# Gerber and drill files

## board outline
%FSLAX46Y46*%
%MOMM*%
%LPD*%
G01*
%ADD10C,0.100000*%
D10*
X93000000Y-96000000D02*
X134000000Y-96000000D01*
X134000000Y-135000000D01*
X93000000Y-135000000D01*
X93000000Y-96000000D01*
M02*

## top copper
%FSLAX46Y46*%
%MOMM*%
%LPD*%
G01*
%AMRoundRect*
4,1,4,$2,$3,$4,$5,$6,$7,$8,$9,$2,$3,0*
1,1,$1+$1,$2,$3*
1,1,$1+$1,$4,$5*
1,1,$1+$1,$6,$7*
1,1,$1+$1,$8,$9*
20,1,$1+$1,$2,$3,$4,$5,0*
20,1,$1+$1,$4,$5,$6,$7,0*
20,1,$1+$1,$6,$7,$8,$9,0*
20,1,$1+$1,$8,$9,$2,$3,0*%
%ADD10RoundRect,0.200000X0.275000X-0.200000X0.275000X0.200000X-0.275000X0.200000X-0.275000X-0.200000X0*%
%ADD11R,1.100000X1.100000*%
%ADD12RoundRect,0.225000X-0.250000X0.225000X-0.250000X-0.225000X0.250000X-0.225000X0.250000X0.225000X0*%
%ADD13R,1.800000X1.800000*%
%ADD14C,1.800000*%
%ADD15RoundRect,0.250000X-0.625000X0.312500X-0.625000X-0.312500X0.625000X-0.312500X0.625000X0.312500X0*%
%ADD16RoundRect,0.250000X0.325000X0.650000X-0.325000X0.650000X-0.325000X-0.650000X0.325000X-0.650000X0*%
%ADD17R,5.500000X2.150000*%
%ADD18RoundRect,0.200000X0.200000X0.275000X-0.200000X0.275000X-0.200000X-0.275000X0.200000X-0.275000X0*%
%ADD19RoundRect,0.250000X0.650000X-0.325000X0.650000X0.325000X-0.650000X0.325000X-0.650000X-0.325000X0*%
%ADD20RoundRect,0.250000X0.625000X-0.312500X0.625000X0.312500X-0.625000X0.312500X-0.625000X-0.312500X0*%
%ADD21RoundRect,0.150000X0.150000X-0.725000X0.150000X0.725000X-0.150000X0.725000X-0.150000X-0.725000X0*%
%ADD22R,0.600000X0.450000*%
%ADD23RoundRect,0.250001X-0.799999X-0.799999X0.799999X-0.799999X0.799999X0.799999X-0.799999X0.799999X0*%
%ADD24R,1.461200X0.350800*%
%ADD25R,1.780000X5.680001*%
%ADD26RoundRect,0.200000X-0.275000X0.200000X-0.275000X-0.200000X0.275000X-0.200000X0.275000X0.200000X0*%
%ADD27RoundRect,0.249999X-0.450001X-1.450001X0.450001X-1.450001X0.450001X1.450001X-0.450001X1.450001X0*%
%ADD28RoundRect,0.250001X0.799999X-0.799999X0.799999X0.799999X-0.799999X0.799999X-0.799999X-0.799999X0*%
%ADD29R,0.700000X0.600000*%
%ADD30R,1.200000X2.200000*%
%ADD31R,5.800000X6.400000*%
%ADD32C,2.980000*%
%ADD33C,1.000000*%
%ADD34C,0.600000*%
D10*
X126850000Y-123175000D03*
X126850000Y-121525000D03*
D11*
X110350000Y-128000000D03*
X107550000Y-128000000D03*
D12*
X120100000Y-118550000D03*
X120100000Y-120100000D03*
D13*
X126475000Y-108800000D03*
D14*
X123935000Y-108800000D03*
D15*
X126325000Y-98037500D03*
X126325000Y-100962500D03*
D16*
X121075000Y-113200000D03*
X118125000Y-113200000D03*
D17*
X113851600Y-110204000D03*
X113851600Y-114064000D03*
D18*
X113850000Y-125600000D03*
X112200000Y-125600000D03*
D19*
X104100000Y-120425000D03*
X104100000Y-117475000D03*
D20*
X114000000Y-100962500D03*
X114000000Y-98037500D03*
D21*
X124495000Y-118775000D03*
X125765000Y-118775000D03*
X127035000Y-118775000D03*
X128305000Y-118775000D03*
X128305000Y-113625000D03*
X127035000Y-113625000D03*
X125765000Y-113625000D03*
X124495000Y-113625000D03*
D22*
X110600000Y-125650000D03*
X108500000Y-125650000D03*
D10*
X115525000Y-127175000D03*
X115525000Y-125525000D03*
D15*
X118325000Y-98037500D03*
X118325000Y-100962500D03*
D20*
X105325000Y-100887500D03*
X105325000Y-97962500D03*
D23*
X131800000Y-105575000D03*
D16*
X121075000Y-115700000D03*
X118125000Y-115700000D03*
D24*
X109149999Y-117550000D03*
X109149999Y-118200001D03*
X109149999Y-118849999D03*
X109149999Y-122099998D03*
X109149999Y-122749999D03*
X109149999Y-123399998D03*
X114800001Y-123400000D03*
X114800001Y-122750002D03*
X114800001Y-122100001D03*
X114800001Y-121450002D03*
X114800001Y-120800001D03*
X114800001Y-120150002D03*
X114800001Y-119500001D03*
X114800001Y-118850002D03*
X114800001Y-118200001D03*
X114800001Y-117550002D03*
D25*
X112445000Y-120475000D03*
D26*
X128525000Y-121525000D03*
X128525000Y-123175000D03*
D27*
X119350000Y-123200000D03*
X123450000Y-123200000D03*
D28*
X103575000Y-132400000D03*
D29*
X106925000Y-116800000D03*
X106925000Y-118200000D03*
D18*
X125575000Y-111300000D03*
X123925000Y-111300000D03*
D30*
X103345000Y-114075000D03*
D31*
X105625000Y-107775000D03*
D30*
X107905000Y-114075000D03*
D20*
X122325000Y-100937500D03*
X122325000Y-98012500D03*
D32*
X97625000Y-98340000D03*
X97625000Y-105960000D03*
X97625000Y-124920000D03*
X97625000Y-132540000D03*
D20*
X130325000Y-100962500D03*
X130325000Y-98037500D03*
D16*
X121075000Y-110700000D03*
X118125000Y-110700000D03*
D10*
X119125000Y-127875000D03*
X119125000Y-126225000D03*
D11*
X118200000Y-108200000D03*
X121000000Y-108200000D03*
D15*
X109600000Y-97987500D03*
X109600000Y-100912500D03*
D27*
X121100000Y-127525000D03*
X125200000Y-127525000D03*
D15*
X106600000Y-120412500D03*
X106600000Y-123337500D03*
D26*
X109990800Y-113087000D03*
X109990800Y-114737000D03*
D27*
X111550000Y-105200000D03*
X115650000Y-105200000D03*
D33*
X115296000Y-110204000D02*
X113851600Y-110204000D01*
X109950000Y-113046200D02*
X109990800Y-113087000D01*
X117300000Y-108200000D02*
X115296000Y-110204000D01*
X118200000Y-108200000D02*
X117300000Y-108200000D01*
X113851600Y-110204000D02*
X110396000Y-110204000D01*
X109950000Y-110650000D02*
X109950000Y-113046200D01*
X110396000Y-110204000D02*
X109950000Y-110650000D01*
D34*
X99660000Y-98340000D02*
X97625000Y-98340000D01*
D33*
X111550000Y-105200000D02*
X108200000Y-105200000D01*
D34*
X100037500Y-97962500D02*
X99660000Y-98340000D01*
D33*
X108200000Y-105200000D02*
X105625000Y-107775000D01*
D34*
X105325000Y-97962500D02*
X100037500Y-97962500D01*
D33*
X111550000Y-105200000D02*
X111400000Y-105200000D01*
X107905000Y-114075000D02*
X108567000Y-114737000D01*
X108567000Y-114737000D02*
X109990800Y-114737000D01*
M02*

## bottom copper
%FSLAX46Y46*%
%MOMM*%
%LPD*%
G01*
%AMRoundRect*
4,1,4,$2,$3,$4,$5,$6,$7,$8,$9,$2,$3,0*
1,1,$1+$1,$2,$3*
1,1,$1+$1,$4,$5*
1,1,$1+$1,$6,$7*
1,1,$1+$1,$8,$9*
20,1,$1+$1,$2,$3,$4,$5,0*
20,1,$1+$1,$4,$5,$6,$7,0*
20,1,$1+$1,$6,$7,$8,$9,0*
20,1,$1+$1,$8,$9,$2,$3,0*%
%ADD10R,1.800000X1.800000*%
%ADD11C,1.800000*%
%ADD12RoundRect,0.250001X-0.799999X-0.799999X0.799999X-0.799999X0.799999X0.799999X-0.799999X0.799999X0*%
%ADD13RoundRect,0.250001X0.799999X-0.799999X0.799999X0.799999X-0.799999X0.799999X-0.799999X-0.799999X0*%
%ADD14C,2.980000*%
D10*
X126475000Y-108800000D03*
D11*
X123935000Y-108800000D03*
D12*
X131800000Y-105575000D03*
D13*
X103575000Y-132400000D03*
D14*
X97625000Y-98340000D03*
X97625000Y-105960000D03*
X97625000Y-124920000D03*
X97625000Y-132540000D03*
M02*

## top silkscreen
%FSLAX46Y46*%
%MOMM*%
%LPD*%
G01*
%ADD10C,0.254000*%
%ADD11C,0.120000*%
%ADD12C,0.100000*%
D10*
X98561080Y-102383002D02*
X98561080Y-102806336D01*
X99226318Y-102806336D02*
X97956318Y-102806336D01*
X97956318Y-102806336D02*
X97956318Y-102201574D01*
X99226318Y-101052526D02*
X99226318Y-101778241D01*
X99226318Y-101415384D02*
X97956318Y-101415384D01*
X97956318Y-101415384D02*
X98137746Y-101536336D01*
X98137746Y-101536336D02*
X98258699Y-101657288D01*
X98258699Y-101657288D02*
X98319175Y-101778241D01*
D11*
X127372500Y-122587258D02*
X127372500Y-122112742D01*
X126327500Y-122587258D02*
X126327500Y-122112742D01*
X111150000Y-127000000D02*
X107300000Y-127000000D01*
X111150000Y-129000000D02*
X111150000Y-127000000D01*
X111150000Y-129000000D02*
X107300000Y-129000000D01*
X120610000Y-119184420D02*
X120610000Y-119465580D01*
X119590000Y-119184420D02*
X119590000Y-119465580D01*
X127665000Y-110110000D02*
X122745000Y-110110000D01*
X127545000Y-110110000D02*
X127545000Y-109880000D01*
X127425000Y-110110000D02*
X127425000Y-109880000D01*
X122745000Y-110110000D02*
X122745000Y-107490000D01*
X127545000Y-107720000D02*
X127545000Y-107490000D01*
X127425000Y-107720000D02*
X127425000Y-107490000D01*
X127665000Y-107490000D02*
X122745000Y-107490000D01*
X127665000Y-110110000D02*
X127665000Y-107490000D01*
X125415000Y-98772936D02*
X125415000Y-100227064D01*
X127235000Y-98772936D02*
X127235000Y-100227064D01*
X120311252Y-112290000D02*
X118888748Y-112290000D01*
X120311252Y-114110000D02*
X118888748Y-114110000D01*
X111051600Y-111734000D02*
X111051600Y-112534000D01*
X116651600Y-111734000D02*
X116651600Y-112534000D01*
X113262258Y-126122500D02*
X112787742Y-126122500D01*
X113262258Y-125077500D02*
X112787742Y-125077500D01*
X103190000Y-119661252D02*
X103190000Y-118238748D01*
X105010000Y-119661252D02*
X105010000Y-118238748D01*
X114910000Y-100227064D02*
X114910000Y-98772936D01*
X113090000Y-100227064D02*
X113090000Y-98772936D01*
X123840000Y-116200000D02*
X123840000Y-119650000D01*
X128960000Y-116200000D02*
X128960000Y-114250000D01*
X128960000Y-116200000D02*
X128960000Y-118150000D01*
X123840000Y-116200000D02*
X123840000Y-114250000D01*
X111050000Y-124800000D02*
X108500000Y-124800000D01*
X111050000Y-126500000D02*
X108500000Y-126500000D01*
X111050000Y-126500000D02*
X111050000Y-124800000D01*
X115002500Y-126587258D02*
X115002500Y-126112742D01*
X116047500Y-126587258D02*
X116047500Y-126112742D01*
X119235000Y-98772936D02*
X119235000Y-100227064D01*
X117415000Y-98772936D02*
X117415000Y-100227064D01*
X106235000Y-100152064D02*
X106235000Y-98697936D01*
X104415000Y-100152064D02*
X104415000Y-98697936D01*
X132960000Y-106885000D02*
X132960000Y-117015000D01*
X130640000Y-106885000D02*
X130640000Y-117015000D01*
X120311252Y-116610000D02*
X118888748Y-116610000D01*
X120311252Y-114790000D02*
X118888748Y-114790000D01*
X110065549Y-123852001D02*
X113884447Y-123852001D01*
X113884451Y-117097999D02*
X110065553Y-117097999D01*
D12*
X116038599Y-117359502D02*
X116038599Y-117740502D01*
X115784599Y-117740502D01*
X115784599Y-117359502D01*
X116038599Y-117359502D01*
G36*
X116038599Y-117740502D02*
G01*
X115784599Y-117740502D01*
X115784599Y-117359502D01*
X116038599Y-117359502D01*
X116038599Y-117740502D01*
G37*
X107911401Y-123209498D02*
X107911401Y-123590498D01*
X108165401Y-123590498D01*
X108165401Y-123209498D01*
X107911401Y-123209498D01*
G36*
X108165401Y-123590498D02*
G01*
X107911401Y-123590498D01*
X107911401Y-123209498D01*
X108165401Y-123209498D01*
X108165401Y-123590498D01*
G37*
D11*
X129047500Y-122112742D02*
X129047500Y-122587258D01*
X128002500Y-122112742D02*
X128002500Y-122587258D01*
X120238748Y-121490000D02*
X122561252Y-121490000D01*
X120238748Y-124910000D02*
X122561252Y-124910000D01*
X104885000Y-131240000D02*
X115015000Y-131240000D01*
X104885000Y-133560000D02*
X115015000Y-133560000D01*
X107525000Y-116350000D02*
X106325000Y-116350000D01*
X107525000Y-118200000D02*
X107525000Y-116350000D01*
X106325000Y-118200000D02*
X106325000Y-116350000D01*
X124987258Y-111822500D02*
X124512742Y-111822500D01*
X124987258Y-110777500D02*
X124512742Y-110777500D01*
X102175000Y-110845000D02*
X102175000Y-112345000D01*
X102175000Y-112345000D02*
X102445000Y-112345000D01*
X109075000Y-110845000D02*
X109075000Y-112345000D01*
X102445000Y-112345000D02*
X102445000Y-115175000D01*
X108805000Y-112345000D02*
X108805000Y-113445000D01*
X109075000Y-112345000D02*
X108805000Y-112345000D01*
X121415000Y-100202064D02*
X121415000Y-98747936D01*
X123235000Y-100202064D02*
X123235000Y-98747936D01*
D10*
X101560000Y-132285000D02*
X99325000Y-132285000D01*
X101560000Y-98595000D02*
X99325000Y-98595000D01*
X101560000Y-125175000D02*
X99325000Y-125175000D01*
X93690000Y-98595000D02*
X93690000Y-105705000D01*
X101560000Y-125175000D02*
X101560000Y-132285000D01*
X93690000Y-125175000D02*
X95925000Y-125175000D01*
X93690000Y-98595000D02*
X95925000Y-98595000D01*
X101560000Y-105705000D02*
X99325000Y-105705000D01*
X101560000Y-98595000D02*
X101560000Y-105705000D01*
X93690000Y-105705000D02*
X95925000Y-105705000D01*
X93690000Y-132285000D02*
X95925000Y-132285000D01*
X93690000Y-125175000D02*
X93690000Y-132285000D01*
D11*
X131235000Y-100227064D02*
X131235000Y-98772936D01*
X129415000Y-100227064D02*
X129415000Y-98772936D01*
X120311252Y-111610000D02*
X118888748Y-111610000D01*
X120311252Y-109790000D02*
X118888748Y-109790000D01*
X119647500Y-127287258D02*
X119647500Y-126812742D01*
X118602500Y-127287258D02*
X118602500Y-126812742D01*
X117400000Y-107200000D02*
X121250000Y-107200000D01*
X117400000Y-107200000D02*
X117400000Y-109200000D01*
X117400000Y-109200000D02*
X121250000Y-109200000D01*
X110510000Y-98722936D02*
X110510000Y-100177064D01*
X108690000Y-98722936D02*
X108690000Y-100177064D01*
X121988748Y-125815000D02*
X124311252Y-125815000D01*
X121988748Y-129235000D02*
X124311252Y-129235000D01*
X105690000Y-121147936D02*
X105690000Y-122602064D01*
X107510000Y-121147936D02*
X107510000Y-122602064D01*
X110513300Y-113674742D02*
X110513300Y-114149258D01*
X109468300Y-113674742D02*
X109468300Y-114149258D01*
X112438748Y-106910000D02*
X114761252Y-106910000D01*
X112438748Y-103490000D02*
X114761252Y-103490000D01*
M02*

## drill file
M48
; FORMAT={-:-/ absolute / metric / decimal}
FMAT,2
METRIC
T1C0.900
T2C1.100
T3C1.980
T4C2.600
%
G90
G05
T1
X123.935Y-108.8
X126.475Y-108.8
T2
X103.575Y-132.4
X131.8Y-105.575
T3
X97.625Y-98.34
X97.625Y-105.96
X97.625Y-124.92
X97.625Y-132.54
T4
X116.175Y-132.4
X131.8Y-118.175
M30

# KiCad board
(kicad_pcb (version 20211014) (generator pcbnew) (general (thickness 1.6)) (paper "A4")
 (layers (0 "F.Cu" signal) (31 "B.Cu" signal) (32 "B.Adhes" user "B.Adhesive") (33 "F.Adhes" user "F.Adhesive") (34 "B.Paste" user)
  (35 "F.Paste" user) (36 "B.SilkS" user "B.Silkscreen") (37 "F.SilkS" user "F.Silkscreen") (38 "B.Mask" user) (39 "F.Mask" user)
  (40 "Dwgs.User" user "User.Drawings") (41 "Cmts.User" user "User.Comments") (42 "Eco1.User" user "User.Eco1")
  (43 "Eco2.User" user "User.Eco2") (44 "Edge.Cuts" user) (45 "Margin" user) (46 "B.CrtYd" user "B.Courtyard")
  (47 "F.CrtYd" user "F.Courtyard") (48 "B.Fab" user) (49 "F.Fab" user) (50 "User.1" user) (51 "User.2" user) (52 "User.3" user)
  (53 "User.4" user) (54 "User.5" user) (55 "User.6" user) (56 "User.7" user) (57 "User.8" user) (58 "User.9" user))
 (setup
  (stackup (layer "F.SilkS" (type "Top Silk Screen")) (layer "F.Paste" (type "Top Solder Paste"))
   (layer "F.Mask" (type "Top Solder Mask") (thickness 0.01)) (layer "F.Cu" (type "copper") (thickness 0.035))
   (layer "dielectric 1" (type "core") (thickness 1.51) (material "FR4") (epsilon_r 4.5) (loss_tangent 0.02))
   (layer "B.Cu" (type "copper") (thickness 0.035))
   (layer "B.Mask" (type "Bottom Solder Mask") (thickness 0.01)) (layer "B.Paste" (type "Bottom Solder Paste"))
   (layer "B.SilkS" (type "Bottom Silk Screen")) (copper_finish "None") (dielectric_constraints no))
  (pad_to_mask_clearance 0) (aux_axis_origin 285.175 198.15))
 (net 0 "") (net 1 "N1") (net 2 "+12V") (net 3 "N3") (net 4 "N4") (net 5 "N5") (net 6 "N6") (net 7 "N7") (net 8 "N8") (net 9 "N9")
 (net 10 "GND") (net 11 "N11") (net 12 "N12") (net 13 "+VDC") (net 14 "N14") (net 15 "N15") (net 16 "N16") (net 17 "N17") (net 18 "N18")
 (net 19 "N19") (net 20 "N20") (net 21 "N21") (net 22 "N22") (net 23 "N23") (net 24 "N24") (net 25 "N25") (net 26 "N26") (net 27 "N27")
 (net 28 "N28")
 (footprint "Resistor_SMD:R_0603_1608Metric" (layer "F.Cu") (at 126.85 122.35 90)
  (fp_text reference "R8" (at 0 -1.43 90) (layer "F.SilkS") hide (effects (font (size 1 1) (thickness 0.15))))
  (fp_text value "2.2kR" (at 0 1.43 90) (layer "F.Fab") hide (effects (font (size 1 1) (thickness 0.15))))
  (fp_line (start -0.237258 0.5225) (end 0.237258 0.5225) (layer "F.SilkS") (width 0.12))
  (fp_line (start -0.237258 -0.5225) (end 0.237258 -0.5225) (layer "F.SilkS") (width 0.12))
  (pad "1" smd roundrect (at -0.825 0 90) (size 0.8 0.95) (layers "F.Cu" "F.Paste" "F.Mask") (roundrect_rratio 0.25) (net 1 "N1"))
  (pad "2" smd roundrect (at 0.825 0 90) (size 0.8 0.95) (layers "F.Cu" "F.Paste" "F.Mask") (roundrect_rratio 0.25) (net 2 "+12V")))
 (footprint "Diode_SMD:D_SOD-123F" (layer "F.Cu") (at 108.95 128 180)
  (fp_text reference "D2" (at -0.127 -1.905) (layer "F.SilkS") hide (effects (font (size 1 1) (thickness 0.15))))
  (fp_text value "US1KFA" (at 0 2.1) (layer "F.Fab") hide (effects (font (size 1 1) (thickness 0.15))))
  (fp_line (start -2.2 1) (end 1.65 1) (layer "F.SilkS") (width 0.12))
  (fp_line (start -2.2 -1) (end -2.2 1) (layer "F.SilkS") (width 0.12))
  (fp_line (start -2.2 -1) (end 1.65 -1) (layer "F.SilkS") (width 0.12))
  (pad "1" smd rect (at -1.4 0 180) (size 1.1 1.1) (layers "F.Cu" "F.Paste" "F.Mask") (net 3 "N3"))
  (pad "2" smd rect (at 1.4 0 180) (size 1.1 1.1) (layers "F.Cu" "F.Paste" "F.Mask") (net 2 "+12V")))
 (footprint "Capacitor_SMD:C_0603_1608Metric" (layer "F.Cu") (at 120.1 119.325 -90)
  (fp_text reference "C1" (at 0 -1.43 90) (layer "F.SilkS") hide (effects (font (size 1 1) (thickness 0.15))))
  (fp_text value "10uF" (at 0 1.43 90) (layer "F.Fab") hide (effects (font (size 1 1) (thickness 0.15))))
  (fp_line (start -0.14058 -0.51) (end 0.14058 -0.51) (layer "F.SilkS") (width 0.12))
  (fp_line (start -0.14058 0.51) (end 0.14058 0.51) (layer "F.SilkS") (width 0.12))
  (pad "1" smd roundrect (at -0.775 0 270) (size 0.9 0.95) (layers "F.Cu" "F.Paste" "F.Mask") (roundrect_rratio 0.25) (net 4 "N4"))
  (pad "2" smd roundrect (at 0.775 0 270) (size 0.9 0.95) (layers "F.Cu" "F.Paste" "F.Mask") (roundrect_rratio 0.25) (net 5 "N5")))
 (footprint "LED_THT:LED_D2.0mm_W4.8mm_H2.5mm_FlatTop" (layer "F.Cu") (at 126.475 108.8 180)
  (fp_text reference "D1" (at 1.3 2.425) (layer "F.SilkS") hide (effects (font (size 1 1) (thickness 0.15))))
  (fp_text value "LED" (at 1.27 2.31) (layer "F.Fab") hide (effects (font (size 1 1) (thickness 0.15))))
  (fp_line (start -1.19 -1.31) (end 3.73 -1.31) (layer "F.SilkS") (width 0.12))
  (fp_line (start -1.07 -1.31) (end -1.07 -1.08) (layer "F.SilkS") (width 0.12))
  (fp_line (start -0.95 -1.31) (end -0.95 -1.08) (layer "F.SilkS") (width 0.12))
  (fp_line (start 3.73 -1.31) (end 3.73 1.31) (layer "F.SilkS") (width 0.12))
  (fp_line (start -1.07 1.08) (end -1.07 1.31) (layer "F.SilkS") (width 0.12))
  (fp_line (start -0.95 1.08) (end -0.95 1.31) (layer "F.SilkS") (width 0.12))
  (fp_line (start -1.19 1.31) (end 3.73 1.31) (layer "F.SilkS") (width 0.12))
  (fp_line (start -1.19 -1.31) (end -1.19 1.31) (layer "F.SilkS") (width 0.12))
  (pad "1" thru_hole rect (at 0 0 180) (size 1.8 1.8) (drill 0.9) (layers *.Cu *.Mask) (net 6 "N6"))
  (pad "2" thru_hole circle (at 2.54 0 180) (size 1.8 1.8) (drill 0.9) (layers *.Cu *.Mask) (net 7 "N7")))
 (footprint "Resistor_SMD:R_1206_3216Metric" (layer "F.Cu") (at 126.325 99.5 -90)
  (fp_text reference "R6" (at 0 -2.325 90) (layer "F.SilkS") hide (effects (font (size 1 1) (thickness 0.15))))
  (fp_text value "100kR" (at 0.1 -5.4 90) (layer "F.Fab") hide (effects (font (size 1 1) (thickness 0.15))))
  (fp_line (start -0.727064 0.91) (end 0.727064 0.91) (layer "F.SilkS") (width 0.12))
  (fp_line (start -0.727064 -0.91) (end 0.727064 -0.91) (layer "F.SilkS") (width 0.12))
  (pad "1" smd roundrect (at -1.4625 0 270) (size 1.125 1.75) (layers "F.Cu" "F.Paste" "F.Mask") (roundrect_rratio 0.222222) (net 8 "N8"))
  (pad "2" smd roundrect (at 1.4625 0 270) (size 1.125 1.75) (layers "F.Cu" "F.Paste" "F.Mask") (roundrect_rratio 0.222222) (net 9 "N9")))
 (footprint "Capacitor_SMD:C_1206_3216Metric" (layer "F.Cu") (at 119.6 113.2 180)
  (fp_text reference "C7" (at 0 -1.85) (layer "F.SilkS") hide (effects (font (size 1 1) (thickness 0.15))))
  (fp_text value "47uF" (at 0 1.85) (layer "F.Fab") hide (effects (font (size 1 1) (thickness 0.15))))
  (fp_line (start -0.711252 0.91) (end 0.711252 0.91) (layer "F.SilkS") (width 0.12))
  (fp_line (start -0.711252 -0.91) (end 0.711252 -0.91) (layer "F.SilkS") (width 0.12))
  (pad "1" smd roundrect (at -1.475 0 180) (size 1.15 1.8) (layers "F.Cu" "F.Paste" "F.Mask") (roundrect_rratio 0.217391) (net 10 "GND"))
  (pad "2" smd roundrect (at 1.475 0 180) (size 1.15 1.8) (layers "F.Cu" "F.Paste" "F.Mask") (roundrect_rratio 0.217391) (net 2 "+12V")))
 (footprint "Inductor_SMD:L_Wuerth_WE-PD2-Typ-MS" (layer "F.Cu") (at 113.8516 112.134 -90)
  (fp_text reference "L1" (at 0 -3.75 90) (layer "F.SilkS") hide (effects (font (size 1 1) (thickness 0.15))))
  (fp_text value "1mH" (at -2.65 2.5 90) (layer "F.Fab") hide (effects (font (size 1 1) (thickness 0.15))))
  (fp_line (start -0.4 2.8) (end 0.4 2.8) (layer "F.SilkS") (width 0.12))
  (fp_line (start -0.4 -2.8) (end 0.4 -2.8) (layer "F.SilkS") (width 0.12))
  (pad "1" smd rect (at -1.93 0 270) (size 2.15 5.5) (layers "F.Cu" "F.Paste" "F.Mask") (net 5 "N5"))
  (pad "2" smd rect (at 1.93 0 270) (size 2.15 5.5) (layers "F.Cu" "F.Paste" "F.Mask") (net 2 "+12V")))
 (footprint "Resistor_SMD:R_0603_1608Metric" (layer "F.Cu") (at 113.025 125.6 180)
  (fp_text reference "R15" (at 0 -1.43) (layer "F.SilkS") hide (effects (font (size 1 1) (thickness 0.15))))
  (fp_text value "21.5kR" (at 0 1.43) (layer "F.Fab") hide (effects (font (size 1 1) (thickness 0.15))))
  (fp_line (start -0.237258 -0.5225) (end 0.237258 -0.5225) (layer "F.SilkS") (width 0.12))
  (fp_line (start -0.237258 0.5225) (end 0.237258 0.5225) (layer "F.SilkS") (width 0.12))
  (pad "1" smd roundrect (at -0.825 0 180) (size 0.8 0.95) (layers "F.Cu" "F.Paste" "F.Mask") (roundrect_rratio 0.25) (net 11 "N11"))
  (pad "2" smd roundrect (at 0.825 0 180) (size 0.8 0.95) (layers "F.Cu" "F.Paste" "F.Mask") (roundrect_rratio 0.25) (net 3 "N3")))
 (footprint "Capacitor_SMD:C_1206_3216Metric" (layer "F.Cu") (at 104.1 118.95 90)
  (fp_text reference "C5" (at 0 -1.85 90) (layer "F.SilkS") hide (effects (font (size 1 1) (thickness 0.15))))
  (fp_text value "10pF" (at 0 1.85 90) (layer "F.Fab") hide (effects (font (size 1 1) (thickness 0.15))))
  (fp_line (start -0.711252 -0.91) (end 0.711252 -0.91) (layer "F.SilkS") (width 0.12))
  (fp_line (start -0.711252 0.91) (end 0.711252 0.91) (layer "F.SilkS") (width 0.12))
  (pad "1" smd roundrect (at -1.475 0 90) (size 1.15 1.8) (layers "F.Cu" "F.Paste" "F.Mask") (roundrect_rratio 0.217391) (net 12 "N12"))
  (pad "2" smd roundrect (at 1.475 0 90) (size 1.15 1.8) (layers "F.Cu" "F.Paste" "F.Mask") (roundrect_rratio 0.217391) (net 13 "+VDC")))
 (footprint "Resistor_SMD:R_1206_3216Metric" (layer "F.Cu") (at 114 99.5 90)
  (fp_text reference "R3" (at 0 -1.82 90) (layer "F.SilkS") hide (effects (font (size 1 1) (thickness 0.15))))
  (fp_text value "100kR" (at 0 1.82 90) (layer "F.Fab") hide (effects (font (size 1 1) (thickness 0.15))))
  (fp_line (start -0.727064 0.91) (end 0.727064 0.91) (layer "F.SilkS") (width 0.12))
  (fp_line (start -0.727064 -0.91) (end 0.727064 -0.91) (layer "F.SilkS") (width 0.12))
  (pad "1" smd roundrect (at -1.4625 0 90) (size 1.125 1.75) (layers "F.Cu" "F.Paste" "F.Mask") (roundrect_rratio 0.222222) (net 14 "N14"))
  (pad "2" smd roundrect (at 1.4625 0 90) (size 1.125 1.75) (layers "F.Cu" "F.Paste" "F.Mask") (roundrect_rratio 0.222222) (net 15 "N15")))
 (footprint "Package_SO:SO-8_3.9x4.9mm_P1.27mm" (layer "F.Cu") (at 126.4 116.2 90)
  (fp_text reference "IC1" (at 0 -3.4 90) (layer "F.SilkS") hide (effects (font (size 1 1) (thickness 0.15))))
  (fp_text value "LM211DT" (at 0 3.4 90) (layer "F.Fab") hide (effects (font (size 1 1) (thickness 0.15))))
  (fp_line (start 0 -2.56) (end -3.45 -2.56) (layer "F.SilkS") (width 0.12))
  (fp_line (start 0 2.56) (end 1.95 2.56) (layer "F.SilkS") (width 0.12))
  (fp_line (start 0 2.56) (end -1.95 2.56) (layer "F.SilkS") (width 0.12))
  (fp_line (start 0 -2.56) (end 1.95 -2.56) (layer "F.SilkS") (width 0.12))
  (pad "1" smd roundrect (at -2.575 -1.905 90) (size 1.75 0.6) (layers "F.Cu" "F.Paste" "F.Mask") (roundrect_rratio 0.25) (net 10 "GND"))
  (pad "2" smd roundrect (at -2.575 -0.635 90) (size 1.75 0.6) (layers "F.Cu" "F.Paste" "F.Mask") (roundrect_rratio 0.25) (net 1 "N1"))
  (pad "3" smd roundrect (at -2.575 0.635 90) (size 1.75 0.6) (layers "F.Cu" "F.Paste" "F.Mask") (roundrect_rratio 0.25) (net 8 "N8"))
  (pad "4" smd roundrect (at -2.575 1.905 90) (size 1.75 0.6) (layers "F.Cu" "F.Paste" "F.Mask") (roundrect_rratio 0.25) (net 10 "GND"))
  (pad "5" smd roundrect (at 2.575 1.905 90) (size 1.75 0.6) (layers "F.Cu" "F.Paste" "F.Mask") (roundrect_rratio 0.25) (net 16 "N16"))
  (pad "6" smd roundrect (at 2.575 0.635 90) (size 1.75 0.6) (layers "F.Cu" "F.Paste" "F.Mask") (roundrect_rratio 0.25) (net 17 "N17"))
  (pad "7" smd roundrect (at 2.575 -0.635 90) (size 1.75 0.6) (layers "F.Cu" "F.Paste" "F.Mask") (roundrect_rratio 0.25) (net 6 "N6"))
  (pad "8" smd roundrect (at 2.575 -1.905 90) (size 1.75 0.6) (layers "F.Cu" "F.Paste" "F.Mask") (roundrect_rratio 0.25) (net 2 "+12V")))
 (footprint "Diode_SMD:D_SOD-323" (layer "F.Cu") (at 109.55 125.65 180)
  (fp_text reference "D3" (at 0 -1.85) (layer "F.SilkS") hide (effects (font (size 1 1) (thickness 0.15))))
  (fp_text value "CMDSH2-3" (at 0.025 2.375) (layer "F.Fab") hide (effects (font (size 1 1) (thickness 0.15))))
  (fp_line (start -1.5 0.85) (end 1.05 0.85) (layer "F.SilkS") (width 0.12))
  (fp_line (start -1.5 -0.85) (end 1.05 -0.85) (layer "F.SilkS") (width 0.12))
  (fp_line (start -1.5 -0.85) (end -1.5 0.85) (layer "F.SilkS") (width 0.12))
  (pad "1" smd rect (at -1.05 0 180) (size 0.6 0.45) (layers "F.Cu" "F.Paste" "F.Mask") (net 3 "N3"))
  (pad "2" smd rect (at 1.05 0 180) (size 0.6 0.45) (layers "F.Cu" "F.Paste" "F.Mask") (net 4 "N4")))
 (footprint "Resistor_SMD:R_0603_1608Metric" (layer "F.Cu") (at 115.525 126.35 90)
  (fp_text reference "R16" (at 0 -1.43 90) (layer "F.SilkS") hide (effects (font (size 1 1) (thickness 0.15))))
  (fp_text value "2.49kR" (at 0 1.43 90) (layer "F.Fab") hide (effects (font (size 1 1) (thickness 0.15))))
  (fp_line (start -0.237258 -0.5225) (end 0.237258 -0.5225) (layer "F.SilkS") (width 0.12))
  (fp_line (start -0.237258 0.5225) (end 0.237258 0.5225) (layer "F.SilkS") (width 0.12))
  (pad "1" smd roundrect (at -0.825 0 90) (size 0.8 0.95) (layers "F.Cu" "F.Paste" "F.Mask") (roundrect_rratio 0.25) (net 5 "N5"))
  (pad "2" smd roundrect (at 0.825 0 90) (size 0.8 0.95) (layers "F.Cu" "F.Paste" "F.Mask") (roundrect_rratio 0.25) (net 11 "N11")))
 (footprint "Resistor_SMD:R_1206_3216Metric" (layer "F.Cu") (at 118.325 99.5 -90)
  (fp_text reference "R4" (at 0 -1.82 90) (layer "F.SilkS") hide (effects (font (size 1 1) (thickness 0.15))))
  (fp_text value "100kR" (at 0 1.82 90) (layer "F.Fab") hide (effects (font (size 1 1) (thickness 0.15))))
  (fp_line (start -0.727064 -0.91) (end 0.727064 -0.91) (layer "F.SilkS") (width 0.12))
  (fp_line (start -0.727064 0.91) (end 0.727064 0.91) (layer "F.SilkS") (width 0.12))
  (pad "1" smd roundrect (at -1.4625 0 270) (size 1.125 1.75) (layers "F.Cu" "F.Paste" "F.Mask") (roundrect_rratio 0.222222) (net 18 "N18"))
  (pad "2" smd roundrect (at 1.4625 0 270) (size 1.125 1.75) (layers "F.Cu" "F.Paste" "F.Mask") (roundrect_rratio 0.222222) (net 14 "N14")))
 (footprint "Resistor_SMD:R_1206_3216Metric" (layer "F.Cu") (at 105.325 99.425 90)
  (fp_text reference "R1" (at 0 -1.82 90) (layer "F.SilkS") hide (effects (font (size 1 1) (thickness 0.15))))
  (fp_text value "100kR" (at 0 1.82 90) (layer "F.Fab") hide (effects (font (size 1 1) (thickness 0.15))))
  (fp_line (start -0.727064 0.91) (end 0.727064 0.91) (layer "F.SilkS") (width 0.12))
  (fp_line (start -0.727064 -0.91) (end 0.727064 -0.91) (layer "F.SilkS") (width 0.12))
  (pad "1" smd roundrect (at -1.4625 0 90) (size 1.125 1.75) (layers "F.Cu" "F.Paste" "F.Mask") (roundrect_rratio 0.222222) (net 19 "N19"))
  (pad "2" smd roundrect (at 1.4625 0 90) (size 1.125 1.75) (layers "F.Cu" "F.Paste" "F.Mask") (roundrect_rratio 0.222222) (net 13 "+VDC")))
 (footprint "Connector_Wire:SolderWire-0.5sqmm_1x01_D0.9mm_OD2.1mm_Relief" (layer "F.Cu") (at 131.8 105.575)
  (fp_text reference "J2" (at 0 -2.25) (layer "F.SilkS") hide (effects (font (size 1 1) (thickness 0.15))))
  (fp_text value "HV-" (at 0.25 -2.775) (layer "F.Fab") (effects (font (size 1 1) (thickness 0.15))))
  (fp_line (start 1.16 1.31) (end 1.16 11.44) (layer "F.SilkS") (width 0.12))
  (fp_line (start -1.16 1.31) (end -1.16 11.44) (layer "F.SilkS") (width 0.12))
  (pad "" np_thru_hole circle (at 0 12.6) (size 2.6 2.6) (drill 2.6) (layers *.Cu *.Mask))
  (pad "1" thru_hole roundrect (at 0 0) (size 2.1 2.1) (drill 1.1) (layers *.Cu *.Mask) (roundrect_rratio 0.119048) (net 10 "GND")))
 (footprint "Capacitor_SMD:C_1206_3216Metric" (layer "F.Cu") (at 119.6 115.7 180)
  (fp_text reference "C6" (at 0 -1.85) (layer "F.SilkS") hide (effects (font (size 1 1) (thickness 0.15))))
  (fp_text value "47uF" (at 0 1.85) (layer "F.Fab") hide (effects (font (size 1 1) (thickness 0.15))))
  (fp_line (start -0.711252 -0.91) (end 0.711252 -0.91) (layer "F.SilkS") (width 0.12))
  (fp_line (start -0.711252 0.91) (end 0.711252 0.91) (layer "F.SilkS") (width 0.12))
  (pad "1" smd roundrect (at -1.475 0 180) (size 1.15 1.8) (layers "F.Cu" "F.Paste" "F.Mask") (roundrect_rratio 0.217391) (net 10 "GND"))
  (pad "2" smd roundrect (at 1.475 0 180) (size 1.15 1.8) (layers "F.Cu" "F.Paste" "F.Mask") (roundrect_rratio 0.217391) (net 2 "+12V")))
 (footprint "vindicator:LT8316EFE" (layer "F.Cu") (at 111.975 120.475)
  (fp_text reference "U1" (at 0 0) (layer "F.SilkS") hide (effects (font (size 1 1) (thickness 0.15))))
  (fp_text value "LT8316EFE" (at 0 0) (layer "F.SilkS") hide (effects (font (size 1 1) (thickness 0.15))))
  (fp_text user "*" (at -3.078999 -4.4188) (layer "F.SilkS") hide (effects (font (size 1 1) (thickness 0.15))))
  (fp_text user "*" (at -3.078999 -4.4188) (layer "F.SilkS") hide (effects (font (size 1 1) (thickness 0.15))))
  (fp_line (start -1.909451 3.377001) (end 1.909447 3.377001) (layer "F.SilkS") (width 0.12))
  (fp_line (start 1.909451 -3.377001) (end -1.909447 -3.377001) (layer "F.SilkS") (width 0.12))
  (fp_poly
   (pts (xy 4.063599 -3.115498) (xy 4.063599 -2.734498) (xy 3.809599 -2.734498) (xy 3.809599 -3.115498)) (layer "F.SilkS") (width 0.1)
   (fill solid))
  (fp_poly
   (pts (xy -4.063599 2.734498) (xy -4.063599 3.115498) (xy -3.809599 3.115498) (xy -3.809599 2.734498)) (layer "F.SilkS") (width 0.1)
   (fill solid))
  (pad "1" smd rect (at -2.825001 -2.925) (size 1.4612 0.3508) (layers "F.Cu" "F.Paste" "F.Mask") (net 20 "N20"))
  (pad "2" smd rect (at -2.825001 -2.274999) (size 1.4612 0.3508) (layers "F.Cu" "F.Paste" "F.Mask") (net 20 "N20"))
  (pad "3" smd rect (at -2.825001 -1.625001) (size 1.4612 0.3508) (layers "F.Cu" "F.Paste" "F.Mask") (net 20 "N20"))
  (pad "8" smd rect (at -2.825001 1.624998) (size 1.4612 0.3508) (layers "F.Cu" "F.Paste" "F.Mask") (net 4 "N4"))
  (pad "9" smd rect (at -2.825001 2.274999) (size 1.4612 0.3508) (layers "F.Cu" "F.Paste" "F.Mask") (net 4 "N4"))
  (pad "10" smd rect (at -2.825001 2.924998) (size 1.4612 0.3508) (layers "F.Cu" "F.Paste" "F.Mask") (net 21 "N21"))
  (pad "11" smd rect (at 2.825001 2.925) (size 1.4612 0.3508) (layers "F.Cu" "F.Paste" "F.Mask") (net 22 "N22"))
  (pad "12" smd rect (at 2.825001 2.275002) (size 1.4612 0.3508) (layers "F.Cu" "F.Paste" "F.Mask") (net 11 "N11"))
  (pad "13" smd rect (at 2.825001 1.625001) (size 1.4612 0.3508) (layers "F.Cu" "F.Paste" "F.Mask") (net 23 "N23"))
  (pad "14" smd rect (at 2.825001 0.975002) (size 1.4612 0.3508) (layers "F.Cu" "F.Paste" "F.Mask") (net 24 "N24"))
  (pad "15" smd rect (at 2.825001 0.325001) (size 1.4612 0.3508) (layers "F.Cu" "F.Paste" "F.Mask") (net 5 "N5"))
  (pad "16" smd rect (at 2.825001 -0.324998) (size 1.4612 0.3508) (layers "F.Cu" "F.Paste" "F.Mask") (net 5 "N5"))
  (pad "17" smd rect (at 2.825001 -0.974999) (size 1.4612 0.3508) (layers "F.Cu" "F.Paste" "F.Mask") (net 4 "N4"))
  (pad "18" smd rect (at 2.825001 -1.624998) (size 1.4612 0.3508) (layers "F.Cu" "F.Paste" "F.Mask") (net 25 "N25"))
  (pad "19" smd rect (at 2.825001 -2.274999) (size 1.4612 0.3508) (layers "F.Cu" "F.Paste" "F.Mask") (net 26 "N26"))
  (pad "20" smd rect (at 2.825001 -2.924998) (size 1.4612 0.3508) (layers "F.Cu" "F.Paste" "F.Mask") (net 5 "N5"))
  (pad "EPAD" smd rect (at 0.47 0) (size 1.78 5.680001) (layers "F.Cu" "F.Paste" "F.Mask") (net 10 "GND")))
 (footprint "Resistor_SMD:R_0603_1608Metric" (layer "F.Cu") (at 128.525 122.35 -90)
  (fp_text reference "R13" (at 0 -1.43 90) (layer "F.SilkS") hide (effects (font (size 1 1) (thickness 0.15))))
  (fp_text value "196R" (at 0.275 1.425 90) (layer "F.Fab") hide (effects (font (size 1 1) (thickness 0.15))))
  (fp_line (start -0.237258 -0.5225) (end 0.237258 -0.5225) (layer "F.SilkS") (width 0.12))
  (fp_line (start -0.237258 0.5225) (end 0.237258 0.5225) (layer "F.SilkS") (width 0.12))
  (pad "1" smd roundrect (at -0.825 0 270) (size 0.8 0.95) (layers "F.Cu" "F.Paste" "F.Mask") (roundrect_rratio 0.25) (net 10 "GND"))
  (pad "2" smd roundrect (at 0.825 0 270) (size 0.8 0.95) (layers "F.Cu" "F.Paste" "F.Mask") (roundrect_rratio 0.25) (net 1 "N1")))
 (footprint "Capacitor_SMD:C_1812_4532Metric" (layer "F.Cu") (at 121.4 123.2)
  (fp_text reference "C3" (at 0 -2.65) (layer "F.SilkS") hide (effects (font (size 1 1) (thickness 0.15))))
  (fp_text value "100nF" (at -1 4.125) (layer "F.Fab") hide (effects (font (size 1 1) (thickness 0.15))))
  (fp_line (start -1.161252 -1.71) (end 1.161252 -1.71) (layer "F.SilkS") (width 0.12))
  (fp_line (start -1.161252 1.71) (end 1.161252 1.71) (layer "F.SilkS") (width 0.12))
  (pad "1" smd roundrect (at -2.05 0) (size 1.4 3.4) (layers "F.Cu" "F.Paste" "F.Mask") (roundrect_rratio 0.178571) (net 24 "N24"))
  (pad "2" smd roundrect (at 2.05 0) (size 1.4 3.4) (layers "F.Cu" "F.Paste" "F.Mask") (roundrect_rratio 0.178571) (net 5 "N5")))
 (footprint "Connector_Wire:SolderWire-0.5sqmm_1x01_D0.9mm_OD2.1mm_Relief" (layer "F.Cu") (at 103.575 132.4 90)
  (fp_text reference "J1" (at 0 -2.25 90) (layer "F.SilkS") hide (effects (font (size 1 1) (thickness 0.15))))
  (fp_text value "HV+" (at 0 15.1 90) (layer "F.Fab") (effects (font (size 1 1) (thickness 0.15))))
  (fp_line (start 1.16 1.31) (end 1.16 11.44) (layer "F.SilkS") (width 0.12))
  (fp_line (start -1.16 1.31) (end -1.16 11.44) (layer "F.SilkS") (width 0.12))
  (pad "" np_thru_hole circle (at 0 12.6 90) (size 2.6 2.6) (drill 2.6) (layers *.Cu *.Mask))
  (pad "1" thru_hole roundrect (at 0 0 90) (size 2.1 2.1) (drill 1.1) (layers *.Cu *.Mask) (roundrect_rratio 0.119048) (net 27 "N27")))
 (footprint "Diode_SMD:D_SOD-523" (layer "F.Cu") (at 106.925 117.5 -90)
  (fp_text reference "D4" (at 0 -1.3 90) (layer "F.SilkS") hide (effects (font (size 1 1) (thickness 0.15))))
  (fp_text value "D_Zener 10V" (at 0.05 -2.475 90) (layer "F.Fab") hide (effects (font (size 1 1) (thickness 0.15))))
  (fp_line (start -1.15 -0.6) (end -1.15 0.6) (layer "F.SilkS") (width 0.12))
  (fp_line (start 0.7 -0.6) (end -1.15 -0.6) (layer "F.SilkS") (width 0.12))
  (fp_line (start 0.7 0.6) (end -1.15 0.6) (layer "F.SilkS") (width 0.12))
  (pad "1" smd rect (at -0.7 0 90) (size 0.6 0.7) (layers "F.Cu" "F.Paste" "F.Mask") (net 13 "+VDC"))
  (pad "2" smd rect (at 0.7 0 90) (size 0.6 0.7) (layers "F.Cu" "F.Paste" "F.Mask") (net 20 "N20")))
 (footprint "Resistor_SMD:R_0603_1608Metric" (layer "F.Cu") (at 124.75 111.3 180)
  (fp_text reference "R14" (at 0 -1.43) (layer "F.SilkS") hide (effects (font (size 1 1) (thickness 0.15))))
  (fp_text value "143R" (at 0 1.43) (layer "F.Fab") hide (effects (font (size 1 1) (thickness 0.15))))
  (fp_line (start -0.237258 -0.5225) (end 0.237258 -0.5225) (layer "F.SilkS") (width 0.12))
  (fp_line (start -0.237258 0.5225) (end 0.237258 0.5225) (layer "F.SilkS") (width 0.12))
  (pad "1" smd roundrect (at -0.825 0 180) (size 0.8 0.95) (layers "F.Cu" "F.Paste" "F.Mask") (roundrect_rratio 0.25) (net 2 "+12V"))
  (pad "2" smd roundrect (at 0.825 0 180) (size 0.8 0.95) (layers "F.Cu" "F.Paste" "F.Mask") (roundrect_rratio 0.25) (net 7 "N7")))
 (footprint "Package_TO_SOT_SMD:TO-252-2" (layer "F.Cu") (at 105.625 109.875 90)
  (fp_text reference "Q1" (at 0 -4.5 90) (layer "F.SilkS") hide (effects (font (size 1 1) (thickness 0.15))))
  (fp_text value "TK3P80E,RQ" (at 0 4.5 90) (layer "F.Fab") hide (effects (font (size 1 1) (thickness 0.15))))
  (fp_line (start -0.97 -3.45) (end -2.47 -3.45) (layer "F.SilkS") (width 0.12))
  (fp_line (start -2.47 -3.45) (end -2.47 -3.18) (layer "F.SilkS") (width 0.12))
  (fp_line (start -0.97 3.45) (end -2.47 3.45) (layer "F.SilkS") (width 0.12))
  (fp_line (start -2.47 -3.18) (end -5.3 -3.18) (layer "F.SilkS") (width 0.12))
  (fp_line (start -2.47 3.18) (end -3.57 3.18) (layer "F.SilkS") (width 0.12))
  (fp_line (start -2.47 3.45) (end -2.47 3.18) (layer "F.SilkS") (width 0.12))
  (pad "" smd rect (at 3.775 1.525 90) (size 3.05 2.75) (layers "F.Paste"))
  (pad "" smd rect (at 0.425 1.525 90) (size 3.05 2.75) (layers "F.Paste"))
  (pad "" smd rect (at 0.425 -1.525 90) (size 3.05 2.75) (layers "F.Paste"))
  (pad "" smd rect (at 3.775 -1.525 90) (size 3.05 2.75) (layers "F.Paste"))
  (pad "1" smd rect (at -4.2 -2.28 90) (size 2.2 1.2) (layers "F.Cu" "F.Paste" "F.Mask") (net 26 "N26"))
  (pad "2" smd rect (at 2.1 0 90) (size 6.4 5.8) (layers "F.Cu" "F.Mask") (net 13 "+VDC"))
  (pad "3" smd rect (at -4.2 2.28 90) (size 2.2 1.2) (layers "F.Cu" "F.Paste" "F.Mask") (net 25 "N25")))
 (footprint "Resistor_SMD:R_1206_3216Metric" (layer "F.Cu") (at 122.325 99.475 90)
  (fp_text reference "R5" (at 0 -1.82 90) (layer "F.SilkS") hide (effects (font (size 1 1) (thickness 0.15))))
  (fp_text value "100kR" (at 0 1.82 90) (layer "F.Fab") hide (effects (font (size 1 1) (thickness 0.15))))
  (fp_line (start -0.727064 -0.91) (end 0.727064 -0.91) (layer "F.SilkS") (width 0.12))
  (fp_line (start -0.727064 0.91) (end 0.727064 0.91) (layer "F.SilkS") (width 0.12))
  (pad "1" smd roundrect (at -1.4625 0 90) (size 1.125 1.75) (layers "F.Cu" "F.Paste" "F.Mask") (roundrect_rratio 0.222222) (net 9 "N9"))
  (pad "2" smd roundrect (at 1.4625 0 90) (size 1.125 1.75) (layers "F.Cu" "F.Paste" "F.Mask") (roundrect_rratio 0.222222) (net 18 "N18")))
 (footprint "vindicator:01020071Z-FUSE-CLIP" (layer "F.Cu") (at 97.625 102.15 -90)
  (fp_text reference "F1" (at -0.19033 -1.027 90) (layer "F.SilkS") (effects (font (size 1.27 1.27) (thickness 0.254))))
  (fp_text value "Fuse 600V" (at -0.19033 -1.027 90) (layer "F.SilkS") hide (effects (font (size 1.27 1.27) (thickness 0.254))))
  (fp_line (start 30.135 -3.935) (end 30.135 -1.7) (layer "F.SilkS") (width 0.254))
  (fp_line (start -3.555 -3.935) (end -3.555 -1.7) (layer "F.SilkS") (width 0.254))
  (fp_line (start 23.025 -3.935) (end 23.025 -1.7) (layer "F.SilkS") (width 0.254))
  (fp_line (start -3.555 3.935) (end 3.555 3.935) (layer "F.SilkS") (width 0.254))
  (fp_line (start 23.025 -3.935) (end 30.135 -3.935) (layer "F.SilkS") (width 0.254))
  (fp_line (start 23.025 3.935) (end 23.025 1.7) (layer "F.SilkS") (width 0.254))
  (fp_line (start -3.555 3.935) (end -3.555 1.7) (layer "F.SilkS") (width 0.254))
  (fp_line (start 3.555 -3.935) (end 3.555 -1.7) (layer "F.SilkS") (width 0.254))
  (fp_line (start -3.555 -3.935) (end 3.555 -3.935) (layer "F.SilkS") (width 0.254))
  (fp_line (start 3.555 3.935) (end 3.555 1.7) (layer "F.SilkS") (width 0.254))
  (fp_line (start 30.135 3.935) (end 30.135 1.7) (layer "F.SilkS") (width 0.254))
  (fp_line (start 23.025 3.935) (end 30.135 3.935) (layer "F.SilkS") (width 0.254))
  (pad "1" thru_hole circle (at -3.81 0 270) (size 2.98 2.98) (drill 1.98) (layers *.Cu *.Mask) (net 13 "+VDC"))
  (pad "1" thru_hole circle (at 3.81 0 270) (size 2.98 2.98) (drill 1.98) (layers *.Cu *.Mask) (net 13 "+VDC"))
  (pad "2" thru_hole circle (at 22.77 0 270) (size 2.98 2.98) (drill 1.98) (layers *.Cu *.Mask) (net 27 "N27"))
  (pad "2" thru_hole circle (at 30.39 0 270) (size 2.98 2.98) (drill 1.98) (layers *.Cu *.Mask) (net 27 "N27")))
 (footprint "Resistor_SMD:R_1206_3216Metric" (layer "F.Cu") (at 130.325 99.5 90)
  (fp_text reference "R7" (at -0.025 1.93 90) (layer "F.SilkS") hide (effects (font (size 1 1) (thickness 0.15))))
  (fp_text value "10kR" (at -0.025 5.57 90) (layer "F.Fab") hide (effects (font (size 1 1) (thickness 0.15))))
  (fp_line (start -0.727064 0.91) (end 0.727064 0.91) (layer "F.SilkS") (width 0.12))
  (fp_line (start -0.727064 -0.91) (end 0.727064 -0.91) (layer "F.SilkS") (width 0.12))
  (pad "1" smd roundrect (at -1.4625 0 90) (size 1.125 1.75) (layers "F.Cu" "F.Paste" "F.Mask") (roundrect_rratio 0.222222) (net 10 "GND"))
  (pad "2" smd roundrect (at 1.4625 0 90) (size 1.125 1.75) (layers "F.Cu" "F.Paste" "F.Mask") (roundrect_rratio 0.222222) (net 8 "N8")))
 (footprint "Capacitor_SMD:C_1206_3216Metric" (layer "F.Cu") (at 119.6 110.7 180)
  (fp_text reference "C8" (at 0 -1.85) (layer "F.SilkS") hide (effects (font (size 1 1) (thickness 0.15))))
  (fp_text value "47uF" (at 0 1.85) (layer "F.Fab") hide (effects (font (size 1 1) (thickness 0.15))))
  (fp_line (start -0.711252 -0.91) (end 0.711252 -0.91) (layer "F.SilkS") (width 0.12))
  (fp_line (start -0.711252 0.91) (end 0.711252 0.91) (layer "F.SilkS") (width 0.12))
  (pad "1" smd roundrect (at -1.475 0 180) (size 1.15 1.8) (layers "F.Cu" "F.Paste" "F.Mask") (roundrect_rratio 0.217391) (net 10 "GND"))
  (pad "2" smd roundrect (at 1.475 0 180) (size 1.15 1.8) (layers "F.Cu" "F.Paste" "F.Mask") (roundrect_rratio 0.217391) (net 2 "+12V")))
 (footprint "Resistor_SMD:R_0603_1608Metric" (layer "F.Cu") (at 119.125 127.05 90)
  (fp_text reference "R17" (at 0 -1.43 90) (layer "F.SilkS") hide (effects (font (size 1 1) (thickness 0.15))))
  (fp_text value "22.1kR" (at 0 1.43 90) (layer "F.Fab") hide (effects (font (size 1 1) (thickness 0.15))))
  (fp_line (start -0.237258 0.5225) (end 0.237258 0.5225) (layer "F.SilkS") (width 0.12))
  (fp_line (start -0.237258 -0.5225) (end 0.237258 -0.5225) (layer "F.SilkS") (width 0.12))
  (pad "1" smd roundrect (at -0.825 0 90) (size 0.8 0.95) (layers "F.Cu" "F.Paste" "F.Mask") (roundrect_rratio 0.25) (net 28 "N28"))
  (pad "2" smd roundrect (at 0.825 0 90) (size 0.8 0.95) (layers "F.Cu" "F.Paste" "F.Mask") (roundrect_rratio 0.25) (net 23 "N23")))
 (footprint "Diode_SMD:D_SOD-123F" (layer "F.Cu") (at 119.6 108.2)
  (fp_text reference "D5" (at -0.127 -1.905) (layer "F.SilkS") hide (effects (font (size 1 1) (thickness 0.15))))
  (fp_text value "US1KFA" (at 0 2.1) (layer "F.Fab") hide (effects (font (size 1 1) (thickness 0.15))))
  (fp_line (start -2.2 -1) (end 1.65 -1) (layer "F.SilkS") (width 0.12))
  (fp_line (start -2.2 -1) (end -2.2 1) (layer "F.SilkS") (width 0.12))
  (fp_line (start -2.2 1) (end 1.65 1) (layer "F.SilkS") (width 0.12))
  (pad "1" smd rect (at -1.4 0) (size 1.1 1.1) (layers "F.Cu" "F.Paste" "F.Mask") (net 5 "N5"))
  (pad "2" smd rect (at 1.4 0) (size 1.1 1.1) (layers "F.Cu" "F.Paste" "F.Mask") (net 10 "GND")))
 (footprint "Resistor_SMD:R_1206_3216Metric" (layer "F.Cu") (at 109.6 99.45 -90)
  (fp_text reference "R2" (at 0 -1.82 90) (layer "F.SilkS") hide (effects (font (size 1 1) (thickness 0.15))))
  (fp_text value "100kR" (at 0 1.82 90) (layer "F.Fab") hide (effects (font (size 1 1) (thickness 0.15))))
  (fp_line (start -0.727064 -0.91) (end 0.727064 -0.91) (layer "F.SilkS") (width 0.12))
  (fp_line (start -0.727064 0.91) (end 0.727064 0.91) (layer "F.SilkS") (width 0.12))
  (pad "1" smd roundrect (at -1.4625 0 270) (size 1.125 1.75) (layers "F.Cu" "F.Paste" "F.Mask") (roundrect_rratio 0.222222) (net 15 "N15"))
  (pad "2" smd roundrect (at 1.4625 0 270) (size 1.125 1.75) (layers "F.Cu" "F.Paste" "F.Mask") (roundrect_rratio 0.222222) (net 19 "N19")))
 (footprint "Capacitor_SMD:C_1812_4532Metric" (layer "F.Cu") (at 123.15 127.525)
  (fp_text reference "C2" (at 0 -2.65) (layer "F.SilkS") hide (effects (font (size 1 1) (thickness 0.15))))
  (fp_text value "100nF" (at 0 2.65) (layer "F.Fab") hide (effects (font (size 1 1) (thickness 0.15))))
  (fp_line (start -1.161252 -1.71) (end 1.161252 -1.71) (layer "F.SilkS") (width 0.12))
  (fp_line (start -1.161252 1.71) (end 1.161252 1.71) (layer "F.SilkS") (width 0.12))
  (pad "1" smd roundrect (at -2.05 0) (size 1.4 3.4) (layers "F.Cu" "F.Paste" "F.Mask") (roundrect_rratio 0.178571) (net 28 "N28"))
  (pad "2" smd roundrect (at 2.05 0) (size 1.4 3.4) (layers "F.Cu" "F.Paste" "F.Mask") (roundrect_rratio 0.178571) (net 5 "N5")))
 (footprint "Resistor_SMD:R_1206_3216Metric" (layer "F.Cu") (at 106.6 121.875 -90)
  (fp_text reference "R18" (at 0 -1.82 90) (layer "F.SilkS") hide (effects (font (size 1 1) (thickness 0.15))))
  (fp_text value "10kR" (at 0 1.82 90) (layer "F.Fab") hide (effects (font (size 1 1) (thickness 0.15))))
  (fp_line (start -0.727064 0.91) (end 0.727064 0.91) (layer "F.SilkS") (width 0.12))
  (fp_line (start -0.727064 -0.91) (end 0.727064 -0.91) (layer "F.SilkS") (width 0.12))
  (pad "1" smd roundrect (at -1.4625 0 270) (size 1.125 1.75) (layers "F.Cu" "F.Paste" "F.Mask") (roundrect_rratio 0.222222) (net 12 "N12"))
  (pad "2" smd roundrect (at 1.4625 0 270) (size 1.125 1.75) (layers "F.Cu" "F.Paste" "F.Mask") (roundrect_rratio 0.222222) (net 21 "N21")))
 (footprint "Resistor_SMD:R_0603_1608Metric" (layer "F.Cu") (at 109.9908 113.912 -90)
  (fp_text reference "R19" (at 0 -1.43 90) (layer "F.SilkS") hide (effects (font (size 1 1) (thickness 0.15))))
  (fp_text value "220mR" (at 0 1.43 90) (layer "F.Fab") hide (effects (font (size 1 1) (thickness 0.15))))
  (fp_line (start -0.237258 -0.5225) (end 0.237258 -0.5225) (layer "F.SilkS") (width 0.12))
  (fp_line (start -0.237258 0.5225) (end 0.237258 0.5225) (layer "F.SilkS") (width 0.12))
  (pad "1" smd roundrect (at -0.825 0 270) (size 0.8 0.95) (layers "F.Cu" "F.Paste" "F.Mask") (roundrect_rratio 0.25) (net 5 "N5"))
  (pad "2" smd roundrect (at 0.825 0 270) (size 0.8 0.95) (layers "F.Cu" "F.Paste" "F.Mask") (roundrect_rratio 0.25) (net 25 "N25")))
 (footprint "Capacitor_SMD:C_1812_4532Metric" (layer "F.Cu") (at 113.6 105.2)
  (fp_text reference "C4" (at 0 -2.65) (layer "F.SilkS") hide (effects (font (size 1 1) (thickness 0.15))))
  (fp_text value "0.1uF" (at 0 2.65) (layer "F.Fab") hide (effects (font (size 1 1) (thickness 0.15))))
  (fp_line (start -1.161252 1.71) (end 1.161252 1.71) (layer "F.SilkS") (width 0.12))
  (fp_line (start -1.161252 -1.71) (end 1.161252 -1.71) (layer "F.SilkS") (width 0.12))
  (pad "1" smd roundrect (at -2.05 0) (size 1.4 3.4) (layers "F.Cu" "F.Paste" "F.Mask") (roundrect_rratio 0.178571) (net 13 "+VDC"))
  (pad "2" smd roundrect (at 2.05 0) (size 1.4 3.4) (layers "F.Cu" "F.Paste" "F.Mask") (roundrect_rratio 0.178571) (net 10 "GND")))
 (gr_rect (start 93 96) (end 134 135) (layer "Edge.Cuts") (width 0.1) (fill none))
 (segment (start 115.296 110.204) (end 113.8516 110.204) (width 1) (layer "F.Cu") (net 5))
 (segment (start 109.95 113.0462) (end 109.9908 113.087) (width 1) (layer "F.Cu") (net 5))
 (segment (start 117.3 108.2) (end 115.296 110.204) (width 1) (layer "F.Cu") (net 5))
 (segment (start 118.2 108.2) (end 117.3 108.2) (width 1) (layer "F.Cu") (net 5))
 (segment (start 113.8516 110.204) (end 110.396 110.204) (width 1) (layer "F.Cu") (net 5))
 (segment (start 109.95 110.65) (end 109.95 113.0462) (width 1) (layer "F.Cu") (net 5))
 (segment (start 110.396 110.204) (end 109.95 110.65) (width 1) (layer "F.Cu") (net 5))
 (segment (start 99.66 98.34) (end 97.625 98.34) (width 0.6) (layer "F.Cu") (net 13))
 (segment (start 111.55 105.2) (end 108.2 105.2) (width 1) (layer "F.Cu") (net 13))
 (segment (start 100.0375 97.9625) (end 99.66 98.34) (width 0.6) (layer "F.Cu") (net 13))
 (segment (start 108.2 105.2) (end 105.625 107.775) (width 1) (layer "F.Cu") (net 13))
 (segment (start 105.325 97.9625) (end 100.0375 97.9625) (width 0.6) (layer "F.Cu") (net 13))
 (segment (start 111.55 105.2) (end 111.4 105.2) (width 1) (layer "F.Cu") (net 13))
 (segment (start 107.905 114.075) (end 108.567 114.737) (width 1) (layer "F.Cu") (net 25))
 (segment (start 108.567 114.737) (end 109.9908 114.737) (width 1) (layer "F.Cu") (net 25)))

